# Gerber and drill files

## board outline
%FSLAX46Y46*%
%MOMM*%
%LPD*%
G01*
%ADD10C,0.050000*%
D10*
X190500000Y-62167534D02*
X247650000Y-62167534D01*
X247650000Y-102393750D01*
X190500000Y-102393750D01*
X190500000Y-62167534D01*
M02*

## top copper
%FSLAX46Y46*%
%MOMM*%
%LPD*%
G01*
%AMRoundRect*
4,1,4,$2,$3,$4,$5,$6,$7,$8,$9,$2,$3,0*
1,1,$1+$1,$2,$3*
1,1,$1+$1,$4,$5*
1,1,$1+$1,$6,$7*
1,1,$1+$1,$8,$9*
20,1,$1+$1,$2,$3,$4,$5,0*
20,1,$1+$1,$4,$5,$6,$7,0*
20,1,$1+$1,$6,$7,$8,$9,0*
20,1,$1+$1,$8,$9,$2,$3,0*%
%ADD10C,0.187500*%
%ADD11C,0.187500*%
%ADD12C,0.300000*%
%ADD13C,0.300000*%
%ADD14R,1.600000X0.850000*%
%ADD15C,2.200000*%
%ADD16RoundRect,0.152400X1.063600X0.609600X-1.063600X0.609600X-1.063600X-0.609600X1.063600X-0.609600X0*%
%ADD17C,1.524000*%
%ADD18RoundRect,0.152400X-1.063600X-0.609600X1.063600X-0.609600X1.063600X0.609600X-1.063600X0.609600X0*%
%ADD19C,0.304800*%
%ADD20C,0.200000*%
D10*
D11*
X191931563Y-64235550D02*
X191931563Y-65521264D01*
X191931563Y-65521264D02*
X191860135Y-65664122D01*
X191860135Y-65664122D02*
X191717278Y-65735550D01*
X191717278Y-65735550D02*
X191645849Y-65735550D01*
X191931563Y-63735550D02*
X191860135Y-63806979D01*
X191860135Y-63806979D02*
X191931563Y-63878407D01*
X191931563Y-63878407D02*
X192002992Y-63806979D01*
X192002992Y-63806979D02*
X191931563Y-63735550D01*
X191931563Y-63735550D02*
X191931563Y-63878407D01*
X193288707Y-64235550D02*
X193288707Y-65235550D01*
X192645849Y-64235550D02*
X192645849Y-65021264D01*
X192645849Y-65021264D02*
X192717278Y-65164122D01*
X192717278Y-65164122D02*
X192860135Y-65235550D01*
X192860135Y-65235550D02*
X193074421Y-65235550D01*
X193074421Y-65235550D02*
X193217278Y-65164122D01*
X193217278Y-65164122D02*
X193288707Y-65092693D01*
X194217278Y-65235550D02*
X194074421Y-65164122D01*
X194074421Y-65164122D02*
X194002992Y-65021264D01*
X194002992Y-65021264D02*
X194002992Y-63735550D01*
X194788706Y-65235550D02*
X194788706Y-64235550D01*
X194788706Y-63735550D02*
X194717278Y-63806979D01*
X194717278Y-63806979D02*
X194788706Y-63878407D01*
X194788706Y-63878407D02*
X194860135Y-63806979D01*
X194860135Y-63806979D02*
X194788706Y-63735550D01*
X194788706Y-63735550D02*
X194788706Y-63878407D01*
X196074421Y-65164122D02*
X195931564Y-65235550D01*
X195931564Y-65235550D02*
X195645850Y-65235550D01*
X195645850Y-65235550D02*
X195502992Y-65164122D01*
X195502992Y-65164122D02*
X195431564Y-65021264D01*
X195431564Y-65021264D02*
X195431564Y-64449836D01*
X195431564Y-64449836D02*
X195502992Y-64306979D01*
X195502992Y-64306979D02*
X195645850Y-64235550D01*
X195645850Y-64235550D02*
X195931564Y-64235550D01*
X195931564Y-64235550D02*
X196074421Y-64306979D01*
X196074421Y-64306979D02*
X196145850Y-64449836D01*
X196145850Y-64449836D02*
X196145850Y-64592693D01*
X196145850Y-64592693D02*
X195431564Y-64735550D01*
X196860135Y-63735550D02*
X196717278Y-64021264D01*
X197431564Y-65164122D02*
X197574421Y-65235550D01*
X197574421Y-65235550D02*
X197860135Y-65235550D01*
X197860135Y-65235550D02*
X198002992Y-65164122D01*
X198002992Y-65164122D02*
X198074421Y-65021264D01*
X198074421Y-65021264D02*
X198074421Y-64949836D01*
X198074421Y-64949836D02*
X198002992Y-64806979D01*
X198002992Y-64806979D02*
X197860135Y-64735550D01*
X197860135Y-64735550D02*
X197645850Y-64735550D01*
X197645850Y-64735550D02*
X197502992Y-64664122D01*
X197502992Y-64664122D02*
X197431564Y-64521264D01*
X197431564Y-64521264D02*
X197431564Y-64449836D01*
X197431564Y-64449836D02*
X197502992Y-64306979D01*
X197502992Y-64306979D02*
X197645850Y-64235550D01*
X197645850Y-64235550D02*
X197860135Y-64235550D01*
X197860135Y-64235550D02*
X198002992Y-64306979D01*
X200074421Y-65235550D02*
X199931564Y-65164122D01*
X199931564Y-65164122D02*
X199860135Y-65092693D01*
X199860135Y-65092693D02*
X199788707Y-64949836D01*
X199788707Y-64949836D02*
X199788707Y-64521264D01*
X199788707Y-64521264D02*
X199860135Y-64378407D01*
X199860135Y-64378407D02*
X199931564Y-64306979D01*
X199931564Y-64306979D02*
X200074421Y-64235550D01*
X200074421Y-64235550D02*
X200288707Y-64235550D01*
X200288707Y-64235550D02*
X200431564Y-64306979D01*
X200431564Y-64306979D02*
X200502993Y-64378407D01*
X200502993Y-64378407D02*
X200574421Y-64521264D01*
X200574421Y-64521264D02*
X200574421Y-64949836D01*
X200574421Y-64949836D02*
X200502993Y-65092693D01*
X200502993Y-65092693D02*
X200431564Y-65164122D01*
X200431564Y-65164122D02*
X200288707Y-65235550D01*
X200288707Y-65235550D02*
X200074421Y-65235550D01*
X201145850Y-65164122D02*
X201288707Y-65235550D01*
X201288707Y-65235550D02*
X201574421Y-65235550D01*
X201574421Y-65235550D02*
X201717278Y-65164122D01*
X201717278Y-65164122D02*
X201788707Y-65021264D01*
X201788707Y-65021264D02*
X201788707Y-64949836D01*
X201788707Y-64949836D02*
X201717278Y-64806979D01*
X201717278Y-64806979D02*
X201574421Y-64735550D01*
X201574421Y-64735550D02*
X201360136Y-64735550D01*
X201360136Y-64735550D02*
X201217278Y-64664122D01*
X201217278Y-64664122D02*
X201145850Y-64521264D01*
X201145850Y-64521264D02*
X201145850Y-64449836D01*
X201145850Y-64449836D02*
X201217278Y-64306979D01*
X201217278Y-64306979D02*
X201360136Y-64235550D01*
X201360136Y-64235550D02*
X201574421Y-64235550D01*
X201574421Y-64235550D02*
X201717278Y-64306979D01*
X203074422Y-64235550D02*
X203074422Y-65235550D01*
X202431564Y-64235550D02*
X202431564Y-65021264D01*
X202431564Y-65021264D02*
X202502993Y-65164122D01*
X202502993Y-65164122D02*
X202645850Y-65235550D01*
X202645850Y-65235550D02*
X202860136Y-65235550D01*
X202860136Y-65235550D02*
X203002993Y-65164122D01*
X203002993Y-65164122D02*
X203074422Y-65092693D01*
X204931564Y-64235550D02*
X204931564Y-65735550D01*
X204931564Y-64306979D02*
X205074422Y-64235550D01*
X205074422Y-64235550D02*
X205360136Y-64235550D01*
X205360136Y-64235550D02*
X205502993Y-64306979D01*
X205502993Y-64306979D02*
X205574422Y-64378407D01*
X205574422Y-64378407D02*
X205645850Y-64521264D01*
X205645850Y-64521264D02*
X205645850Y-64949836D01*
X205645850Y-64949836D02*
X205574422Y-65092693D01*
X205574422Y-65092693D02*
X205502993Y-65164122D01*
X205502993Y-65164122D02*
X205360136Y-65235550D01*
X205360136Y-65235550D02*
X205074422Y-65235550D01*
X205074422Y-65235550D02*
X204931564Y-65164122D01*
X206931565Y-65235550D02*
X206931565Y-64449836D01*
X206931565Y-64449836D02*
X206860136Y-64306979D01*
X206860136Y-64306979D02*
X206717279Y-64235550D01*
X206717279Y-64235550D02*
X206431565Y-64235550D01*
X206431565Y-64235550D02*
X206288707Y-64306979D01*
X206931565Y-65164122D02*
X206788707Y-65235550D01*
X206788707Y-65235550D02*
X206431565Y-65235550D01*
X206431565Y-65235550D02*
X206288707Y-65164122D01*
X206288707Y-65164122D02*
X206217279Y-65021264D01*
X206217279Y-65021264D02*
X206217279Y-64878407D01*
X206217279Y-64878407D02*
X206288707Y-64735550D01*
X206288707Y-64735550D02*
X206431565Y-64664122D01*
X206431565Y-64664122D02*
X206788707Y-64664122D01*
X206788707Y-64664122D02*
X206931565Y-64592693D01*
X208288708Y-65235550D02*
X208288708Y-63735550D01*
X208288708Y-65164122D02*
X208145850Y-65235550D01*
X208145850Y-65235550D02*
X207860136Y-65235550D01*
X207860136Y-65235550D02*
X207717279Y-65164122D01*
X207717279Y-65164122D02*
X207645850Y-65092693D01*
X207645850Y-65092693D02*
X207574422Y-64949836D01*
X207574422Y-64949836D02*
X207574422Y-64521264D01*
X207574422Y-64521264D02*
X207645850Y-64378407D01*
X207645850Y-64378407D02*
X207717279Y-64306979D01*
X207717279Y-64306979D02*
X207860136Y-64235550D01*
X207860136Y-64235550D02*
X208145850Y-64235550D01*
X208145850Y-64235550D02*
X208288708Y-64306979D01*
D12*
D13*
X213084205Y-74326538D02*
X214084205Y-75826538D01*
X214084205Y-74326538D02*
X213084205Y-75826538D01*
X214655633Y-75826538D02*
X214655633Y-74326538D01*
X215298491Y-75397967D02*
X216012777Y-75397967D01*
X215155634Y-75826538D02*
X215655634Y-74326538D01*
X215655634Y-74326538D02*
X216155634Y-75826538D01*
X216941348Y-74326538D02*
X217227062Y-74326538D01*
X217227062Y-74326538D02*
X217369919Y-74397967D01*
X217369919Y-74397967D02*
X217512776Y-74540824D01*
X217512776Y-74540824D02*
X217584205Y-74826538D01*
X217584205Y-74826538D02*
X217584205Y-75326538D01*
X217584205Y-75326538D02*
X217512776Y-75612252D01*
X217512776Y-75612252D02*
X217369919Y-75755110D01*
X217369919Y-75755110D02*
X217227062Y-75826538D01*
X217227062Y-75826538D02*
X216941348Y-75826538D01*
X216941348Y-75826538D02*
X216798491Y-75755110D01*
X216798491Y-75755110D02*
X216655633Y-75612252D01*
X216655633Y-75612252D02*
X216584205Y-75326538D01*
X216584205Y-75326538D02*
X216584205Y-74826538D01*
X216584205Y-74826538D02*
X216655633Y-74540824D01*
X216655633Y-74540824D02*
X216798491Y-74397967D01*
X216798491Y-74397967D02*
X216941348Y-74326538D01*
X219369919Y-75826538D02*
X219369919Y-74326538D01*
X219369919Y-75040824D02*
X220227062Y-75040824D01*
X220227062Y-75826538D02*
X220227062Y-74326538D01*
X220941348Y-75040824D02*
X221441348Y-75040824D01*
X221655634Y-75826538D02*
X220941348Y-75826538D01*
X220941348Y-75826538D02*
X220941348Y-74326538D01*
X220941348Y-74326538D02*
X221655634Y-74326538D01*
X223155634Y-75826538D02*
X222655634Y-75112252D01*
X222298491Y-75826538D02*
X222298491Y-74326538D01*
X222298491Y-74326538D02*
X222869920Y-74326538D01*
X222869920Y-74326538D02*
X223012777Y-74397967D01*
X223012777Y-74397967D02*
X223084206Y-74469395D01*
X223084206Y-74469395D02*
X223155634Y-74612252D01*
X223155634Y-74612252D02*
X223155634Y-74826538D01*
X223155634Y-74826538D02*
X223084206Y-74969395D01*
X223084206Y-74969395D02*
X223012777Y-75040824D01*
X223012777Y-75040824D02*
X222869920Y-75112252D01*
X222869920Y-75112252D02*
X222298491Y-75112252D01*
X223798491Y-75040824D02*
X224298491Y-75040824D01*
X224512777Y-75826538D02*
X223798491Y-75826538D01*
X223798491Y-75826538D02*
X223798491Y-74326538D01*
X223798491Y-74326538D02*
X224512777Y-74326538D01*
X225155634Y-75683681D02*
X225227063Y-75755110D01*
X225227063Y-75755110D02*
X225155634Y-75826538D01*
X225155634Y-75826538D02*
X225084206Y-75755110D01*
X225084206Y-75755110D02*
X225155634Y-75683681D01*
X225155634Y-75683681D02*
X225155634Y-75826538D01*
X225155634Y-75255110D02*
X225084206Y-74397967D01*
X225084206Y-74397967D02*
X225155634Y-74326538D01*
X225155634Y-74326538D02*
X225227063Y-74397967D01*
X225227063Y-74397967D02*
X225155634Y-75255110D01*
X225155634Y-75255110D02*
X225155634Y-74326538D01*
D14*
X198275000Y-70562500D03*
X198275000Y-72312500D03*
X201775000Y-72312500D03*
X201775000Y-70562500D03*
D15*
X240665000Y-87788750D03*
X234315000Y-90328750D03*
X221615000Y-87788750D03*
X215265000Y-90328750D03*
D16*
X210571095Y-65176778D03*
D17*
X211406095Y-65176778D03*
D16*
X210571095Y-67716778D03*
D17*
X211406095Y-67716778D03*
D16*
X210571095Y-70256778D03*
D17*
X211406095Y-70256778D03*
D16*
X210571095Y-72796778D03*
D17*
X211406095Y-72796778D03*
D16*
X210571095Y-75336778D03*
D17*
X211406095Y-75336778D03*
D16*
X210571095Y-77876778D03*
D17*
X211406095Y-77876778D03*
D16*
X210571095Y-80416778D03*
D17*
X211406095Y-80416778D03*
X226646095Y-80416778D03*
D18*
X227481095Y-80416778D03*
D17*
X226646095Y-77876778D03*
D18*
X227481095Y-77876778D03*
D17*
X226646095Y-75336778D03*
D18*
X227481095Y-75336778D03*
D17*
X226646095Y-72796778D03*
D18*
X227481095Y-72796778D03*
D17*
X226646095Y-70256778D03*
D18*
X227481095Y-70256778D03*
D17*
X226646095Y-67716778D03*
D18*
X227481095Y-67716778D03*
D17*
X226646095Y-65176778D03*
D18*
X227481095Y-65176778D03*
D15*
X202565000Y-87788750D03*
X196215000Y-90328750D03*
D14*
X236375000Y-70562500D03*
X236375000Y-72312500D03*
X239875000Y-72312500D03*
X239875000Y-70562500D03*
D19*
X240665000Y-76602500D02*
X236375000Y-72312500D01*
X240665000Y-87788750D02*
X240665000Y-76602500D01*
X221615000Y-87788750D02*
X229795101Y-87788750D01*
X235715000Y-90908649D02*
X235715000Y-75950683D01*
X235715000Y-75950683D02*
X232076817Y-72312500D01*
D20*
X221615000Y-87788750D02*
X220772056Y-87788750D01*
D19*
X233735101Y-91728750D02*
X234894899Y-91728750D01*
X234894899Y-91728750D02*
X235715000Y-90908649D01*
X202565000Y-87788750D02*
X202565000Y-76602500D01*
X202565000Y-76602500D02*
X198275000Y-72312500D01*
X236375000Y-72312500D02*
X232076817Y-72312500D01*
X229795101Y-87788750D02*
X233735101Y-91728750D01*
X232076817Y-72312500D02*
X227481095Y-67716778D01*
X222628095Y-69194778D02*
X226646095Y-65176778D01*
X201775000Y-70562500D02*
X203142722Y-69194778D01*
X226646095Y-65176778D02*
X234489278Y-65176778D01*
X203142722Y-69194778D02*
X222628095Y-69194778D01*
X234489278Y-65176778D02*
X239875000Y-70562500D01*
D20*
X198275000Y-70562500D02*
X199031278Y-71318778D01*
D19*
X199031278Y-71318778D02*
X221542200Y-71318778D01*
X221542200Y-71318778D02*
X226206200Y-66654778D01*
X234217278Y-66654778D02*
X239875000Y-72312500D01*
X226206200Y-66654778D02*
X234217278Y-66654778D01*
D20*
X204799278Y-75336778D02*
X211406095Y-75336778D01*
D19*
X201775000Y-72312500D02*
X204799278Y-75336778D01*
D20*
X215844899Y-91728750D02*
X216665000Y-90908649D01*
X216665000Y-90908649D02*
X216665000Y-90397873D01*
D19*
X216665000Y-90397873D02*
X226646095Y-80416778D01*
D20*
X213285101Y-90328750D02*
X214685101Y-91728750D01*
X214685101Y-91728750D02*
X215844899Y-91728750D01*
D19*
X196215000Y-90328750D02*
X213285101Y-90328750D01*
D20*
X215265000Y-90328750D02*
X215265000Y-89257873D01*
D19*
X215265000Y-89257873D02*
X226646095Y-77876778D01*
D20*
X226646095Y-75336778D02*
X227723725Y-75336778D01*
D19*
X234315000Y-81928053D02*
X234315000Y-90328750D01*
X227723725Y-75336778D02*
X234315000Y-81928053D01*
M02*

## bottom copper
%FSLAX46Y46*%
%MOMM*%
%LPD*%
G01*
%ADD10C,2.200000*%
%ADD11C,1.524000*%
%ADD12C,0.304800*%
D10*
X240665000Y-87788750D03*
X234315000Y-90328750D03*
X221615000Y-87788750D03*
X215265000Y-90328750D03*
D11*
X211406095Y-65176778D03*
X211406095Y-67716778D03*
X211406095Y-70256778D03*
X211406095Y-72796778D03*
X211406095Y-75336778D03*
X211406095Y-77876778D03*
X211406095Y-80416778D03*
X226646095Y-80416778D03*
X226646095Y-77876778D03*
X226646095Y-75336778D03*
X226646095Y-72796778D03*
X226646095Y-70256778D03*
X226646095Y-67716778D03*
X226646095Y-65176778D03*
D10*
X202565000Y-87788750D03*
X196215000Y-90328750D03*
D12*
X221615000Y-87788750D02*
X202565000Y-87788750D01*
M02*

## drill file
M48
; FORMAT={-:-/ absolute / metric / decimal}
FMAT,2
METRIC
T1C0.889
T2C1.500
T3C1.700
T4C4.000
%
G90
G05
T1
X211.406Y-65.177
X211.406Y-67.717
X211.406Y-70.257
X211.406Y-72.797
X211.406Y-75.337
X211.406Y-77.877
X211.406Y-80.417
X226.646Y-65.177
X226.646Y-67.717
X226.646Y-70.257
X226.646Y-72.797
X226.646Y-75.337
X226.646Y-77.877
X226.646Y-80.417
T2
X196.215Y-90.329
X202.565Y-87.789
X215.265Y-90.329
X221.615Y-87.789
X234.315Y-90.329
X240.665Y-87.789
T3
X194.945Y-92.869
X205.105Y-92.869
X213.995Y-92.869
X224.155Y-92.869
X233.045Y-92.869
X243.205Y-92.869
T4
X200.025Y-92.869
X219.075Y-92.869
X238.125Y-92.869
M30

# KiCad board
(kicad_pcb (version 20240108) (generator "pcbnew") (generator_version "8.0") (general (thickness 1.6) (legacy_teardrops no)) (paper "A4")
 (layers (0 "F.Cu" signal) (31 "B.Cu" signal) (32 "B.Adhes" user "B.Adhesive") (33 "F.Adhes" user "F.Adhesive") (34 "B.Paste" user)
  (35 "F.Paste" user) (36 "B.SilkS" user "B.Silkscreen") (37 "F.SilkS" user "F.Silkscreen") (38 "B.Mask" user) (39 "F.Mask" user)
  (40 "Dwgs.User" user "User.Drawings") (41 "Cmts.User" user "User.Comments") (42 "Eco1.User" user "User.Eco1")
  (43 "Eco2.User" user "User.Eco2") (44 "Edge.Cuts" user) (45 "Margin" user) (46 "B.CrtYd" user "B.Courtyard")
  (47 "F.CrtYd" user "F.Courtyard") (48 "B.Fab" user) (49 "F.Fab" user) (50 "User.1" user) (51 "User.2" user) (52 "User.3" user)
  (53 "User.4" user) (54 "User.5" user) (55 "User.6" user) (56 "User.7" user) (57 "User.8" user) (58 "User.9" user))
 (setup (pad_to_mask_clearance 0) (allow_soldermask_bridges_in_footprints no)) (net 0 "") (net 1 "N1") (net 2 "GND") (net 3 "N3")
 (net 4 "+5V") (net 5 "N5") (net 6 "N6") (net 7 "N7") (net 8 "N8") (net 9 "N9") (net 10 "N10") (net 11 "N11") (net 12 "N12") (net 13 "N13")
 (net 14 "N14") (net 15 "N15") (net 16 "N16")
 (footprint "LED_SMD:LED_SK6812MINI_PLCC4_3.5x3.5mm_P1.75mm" (layer "F.Cu") (at 200.025 71.4375)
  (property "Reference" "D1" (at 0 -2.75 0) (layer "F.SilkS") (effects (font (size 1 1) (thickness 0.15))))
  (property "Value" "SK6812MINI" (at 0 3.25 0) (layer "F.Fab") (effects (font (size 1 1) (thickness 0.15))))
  (pad "1" smd rect (at -1.75 -0.875) (size 1.6 0.85) (layers "F.Cu" "F.Paste" "F.Mask") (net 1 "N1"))
  (pad "2" smd rect (at -1.75 0.875) (size 1.6 0.85) (layers "F.Cu" "F.Paste" "F.Mask") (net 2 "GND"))
  (pad "3" smd rect (at 1.75 0.875) (size 1.6 0.85) (layers "F.Cu" "F.Paste" "F.Mask") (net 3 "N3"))
  (pad "4" smd rect (at 1.75 -0.875) (size 1.6 0.85) (layers "F.Cu" "F.Paste" "F.Mask") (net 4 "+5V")))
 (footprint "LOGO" (layer "F.Cu") (at 219.075 76.2)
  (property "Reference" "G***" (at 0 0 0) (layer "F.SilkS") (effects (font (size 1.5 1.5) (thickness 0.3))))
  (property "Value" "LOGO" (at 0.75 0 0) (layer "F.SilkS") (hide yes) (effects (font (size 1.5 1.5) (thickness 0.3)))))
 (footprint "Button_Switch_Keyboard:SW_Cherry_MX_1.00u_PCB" (layer "F.Cu") (at 240.665 87.78875)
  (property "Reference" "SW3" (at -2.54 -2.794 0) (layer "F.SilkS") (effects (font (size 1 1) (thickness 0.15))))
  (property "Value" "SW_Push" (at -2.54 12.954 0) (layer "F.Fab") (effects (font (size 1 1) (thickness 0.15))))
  (pad "" np_thru_hole circle (at -7.62 5.08) (size 1.7 1.7) (drill 1.7) (layers "*.Cu" "*.Mask"))
  (pad "" np_thru_hole circle (at -2.54 5.08) (size 4 4) (drill 4) (layers "*.Cu" "*.Mask"))
  (pad "" np_thru_hole circle (at 2.54 5.08) (size 1.7 1.7) (drill 1.7) (layers "*.Cu" "*.Mask"))
  (pad "1" thru_hole circle (at 0 0) (size 2.2 2.2) (drill 1.5) (layers "*.Cu" "*.Mask") (remove_unused_layers no) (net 2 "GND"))
  (pad "2" thru_hole circle (at -6.35 2.54) (size 2.2 2.2) (drill 1.5) (layers "*.Cu" "*.Mask") (remove_unused_layers no) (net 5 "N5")))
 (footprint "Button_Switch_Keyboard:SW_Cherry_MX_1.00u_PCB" (layer "F.Cu") (at 221.615 87.78875)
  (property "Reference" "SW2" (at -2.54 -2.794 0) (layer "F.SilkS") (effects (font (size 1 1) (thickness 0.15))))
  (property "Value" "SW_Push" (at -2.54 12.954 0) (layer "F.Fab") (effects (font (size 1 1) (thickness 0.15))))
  (pad "" np_thru_hole circle (at -7.62 5.08) (size 1.7 1.7) (drill 1.7) (layers "*.Cu" "*.Mask"))
  (pad "" np_thru_hole circle (at -2.54 5.08) (size 4 4) (drill 4) (layers "*.Cu" "*.Mask"))
  (pad "" np_thru_hole circle (at 2.54 5.08) (size 1.7 1.7) (drill 1.7) (layers "*.Cu" "*.Mask"))
  (pad "1" thru_hole circle (at 0 0) (size 2.2 2.2) (drill 1.5) (layers "*.Cu" "*.Mask") (remove_unused_layers no) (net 2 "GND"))
  (pad "2" thru_hole circle (at -6.35 2.54) (size 2.2 2.2) (drill 1.5) (layers "*.Cu" "*.Mask") (remove_unused_layers no) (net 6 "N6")))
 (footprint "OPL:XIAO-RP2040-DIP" (layer "F.Cu") (at 219.026095 72.796778)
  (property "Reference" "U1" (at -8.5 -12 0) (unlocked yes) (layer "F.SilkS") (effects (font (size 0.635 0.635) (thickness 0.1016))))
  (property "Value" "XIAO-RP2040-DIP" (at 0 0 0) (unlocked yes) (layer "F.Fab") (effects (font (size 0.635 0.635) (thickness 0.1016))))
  (pad "1" smd roundrect (at -8.455 -7.62 180) (size 2.432 1.524) (layers "F.Cu" "F.Mask") (roundrect_rratio 0.1) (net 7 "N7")
   (thermal_bridge_angle 45))
  (pad "1" thru_hole circle (at -7.62 -7.62 180) (size 1.524 1.524) (drill 0.889) (layers "*.Cu" "*.Mask") (remove_unused_layers no)
   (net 7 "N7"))
  (pad "2" smd roundrect (at -8.455 -5.08 180) (size 2.432 1.524) (layers "F.Cu" "F.Mask") (roundrect_rratio 0.1) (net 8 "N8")
   (thermal_bridge_angle 45))
  (pad "2" thru_hole circle (at -7.62 -5.08 180) (size 1.524 1.524) (drill 0.889) (layers "*.Cu" "*.Mask") (remove_unused_layers no)
   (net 8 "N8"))
  (pad "3" smd roundrect (at -8.455 -2.54 180) (size 2.432 1.524) (layers "F.Cu" "F.Mask") (roundrect_rratio 0.1) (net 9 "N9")
   (thermal_bridge_angle 45))
  (pad "3" thru_hole circle (at -7.62 -2.54 180) (size 1.524 1.524) (drill 0.889) (layers "*.Cu" "*.Mask") (remove_unused_layers no)
   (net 9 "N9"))
  (pad "4" smd roundrect (at -8.455 0 180) (size 2.432 1.524) (layers "F.Cu" "F.Mask") (roundrect_rratio 0.1) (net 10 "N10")
   (thermal_bridge_angle 45))
  (pad "4" thru_hole circle (at -7.62 0 180) (size 1.524 1.524) (drill 0.889) (layers "*.Cu" "*.Mask") (remove_unused_layers no)
   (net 10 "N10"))
  (pad "5" smd roundrect (at -8.455 2.54 180) (size 2.432 1.524) (layers "F.Cu" "F.Mask") (roundrect_rratio 0.1) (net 3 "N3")
   (thermal_bridge_angle 45))
  (pad "5" thru_hole circle (at -7.62 2.54 180) (size 1.524 1.524) (drill 0.889) (layers "*.Cu" "*.Mask") (remove_unused_layers no)
   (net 3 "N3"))
  (pad "6" smd roundrect (at -8.455 5.08 180) (size 2.432 1.524) (layers "F.Cu" "F.Mask") (roundrect_rratio 0.1) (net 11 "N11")
   (thermal_bridge_angle 45))
  (pad "6" thru_hole circle (at -7.62 5.08 180) (size 1.524 1.524) (drill 0.889) (layers "*.Cu" "*.Mask") (remove_unused_layers no)
   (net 11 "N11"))
  (pad "7" smd roundrect (at -8.455 7.62 180) (size 2.432 1.524) (layers "F.Cu" "F.Mask") (roundrect_rratio 0.1) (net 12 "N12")
   (thermal_bridge_angle 45))
  (pad "7" thru_hole circle (at -7.62 7.62 180) (size 1.524 1.524) (drill 0.889) (layers "*.Cu" "*.Mask") (remove_unused_layers no)
   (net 12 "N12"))
  (pad "8" thru_hole circle (at 7.62 7.62) (size 1.524 1.524) (drill 0.889) (layers "*.Cu" "*.Mask") (remove_unused_layers no)
   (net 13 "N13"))
  (pad "8" smd roundrect (at 8.455 7.62) (size 2.432 1.524) (layers "F.Cu" "F.Mask") (roundrect_rratio 0.1) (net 13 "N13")
   (thermal_bridge_angle 45))
  (pad "9" thru_hole circle (at 7.62 5.08) (size 1.524 1.524) (drill 0.889) (layers "*.Cu" "*.Mask") (remove_unused_layers no) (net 6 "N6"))
  (pad "9" smd roundrect (at 8.455 5.08) (size 2.432 1.524) (layers "F.Cu" "F.Mask") (roundrect_rratio 0.1) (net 6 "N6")
   (thermal_bridge_angle 45))
  (pad "10" thru_hole circle (at 7.62 2.54) (size 1.524 1.524) (drill 0.889) (layers "*.Cu" "*.Mask") (remove_unused_layers no) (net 5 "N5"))
  (pad "10" smd roundrect (at 8.455 2.54) (size 2.432 1.524) (layers "F.Cu" "F.Mask") (roundrect_rratio 0.1) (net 5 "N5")
   (thermal_bridge_angle 45))
  (pad "11" thru_hole circle (at 7.62 0) (size 1.524 1.524) (drill 0.889) (layers "*.Cu" "*.Mask") (remove_unused_layers no) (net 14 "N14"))
  (pad "11" smd roundrect (at 8.455 0) (size 2.432 1.524) (layers "F.Cu" "F.Mask") (roundrect_rratio 0.1) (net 14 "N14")
   (thermal_bridge_angle 45))
  (pad "12" thru_hole circle (at 7.62 -2.54) (size 1.524 1.524) (drill 0.889) (layers "*.Cu" "*.Mask") (remove_unused_layers no)
   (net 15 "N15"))
  (pad "12" smd roundrect (at 8.455 -2.54) (size 2.432 1.524) (layers "F.Cu" "F.Mask") (roundrect_rratio 0.1) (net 15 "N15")
   (thermal_bridge_angle 45))
  (pad "13" thru_hole circle (at 7.62 -5.08) (size 1.524 1.524) (drill 0.889) (layers "*.Cu" "*.Mask") (remove_unused_layers no)
   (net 2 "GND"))
  (pad "13" smd roundrect (at 8.455 -5.08) (size 2.432 1.524) (layers "F.Cu" "F.Mask") (roundrect_rratio 0.1) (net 2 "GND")
   (thermal_bridge_angle 45))
  (pad "14" thru_hole circle (at 7.62 -7.62) (size 1.524 1.524) (drill 0.889) (layers "*.Cu" "*.Mask") (remove_unused_layers no)
   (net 4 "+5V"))
  (pad "14" smd roundrect (at 8.455 -7.62) (size 2.432 1.524) (layers "F.Cu" "F.Mask") (roundrect_rratio 0.1) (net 4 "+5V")
   (thermal_bridge_angle 45)))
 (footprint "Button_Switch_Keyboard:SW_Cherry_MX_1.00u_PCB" (layer "F.Cu") (at 202.565 87.78875)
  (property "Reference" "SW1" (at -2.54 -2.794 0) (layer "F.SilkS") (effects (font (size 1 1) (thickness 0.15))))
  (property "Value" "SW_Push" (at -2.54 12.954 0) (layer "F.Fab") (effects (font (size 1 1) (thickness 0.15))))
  (pad "" np_thru_hole circle (at -7.62 5.08) (size 1.7 1.7) (drill 1.7) (layers "*.Cu" "*.Mask"))
  (pad "" np_thru_hole circle (at -2.54 5.08) (size 4 4) (drill 4) (layers "*.Cu" "*.Mask"))
  (pad "" np_thru_hole circle (at 2.54 5.08) (size 1.7 1.7) (drill 1.7) (layers "*.Cu" "*.Mask"))
  (pad "1" thru_hole circle (at 0 0) (size 2.2 2.2) (drill 1.5) (layers "*.Cu" "*.Mask") (remove_unused_layers no) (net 2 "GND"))
  (pad "2" thru_hole circle (at -6.35 2.54) (size 2.2 2.2) (drill 1.5) (layers "*.Cu" "*.Mask") (remove_unused_layers no) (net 13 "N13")))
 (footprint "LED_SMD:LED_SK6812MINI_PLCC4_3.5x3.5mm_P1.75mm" (layer "F.Cu") (at 238.125 71.4375)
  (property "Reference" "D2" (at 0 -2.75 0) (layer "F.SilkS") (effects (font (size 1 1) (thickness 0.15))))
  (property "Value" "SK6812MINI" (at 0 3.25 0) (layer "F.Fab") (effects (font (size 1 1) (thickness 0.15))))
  (pad "1" smd rect (at -1.75 -0.875) (size 1.6 0.85) (layers "F.Cu" "F.Paste" "F.Mask") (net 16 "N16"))
  (pad "2" smd rect (at -1.75 0.875) (size 1.6 0.85) (layers "F.Cu" "F.Paste" "F.Mask") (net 2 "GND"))
  (pad "3" smd rect (at 1.75 0.875) (size 1.6 0.85) (layers "F.Cu" "F.Paste" "F.Mask") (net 1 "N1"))
  (pad "4" smd rect (at 1.75 -0.875) (size 1.6 0.85) (layers "F.Cu" "F.Paste" "F.Mask") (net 4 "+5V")))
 (gr_rect (start 190.5 62.167534) (end 247.65 102.39375) (stroke (width 0.05) (type default)) (fill none) (layer "Edge.Cuts"))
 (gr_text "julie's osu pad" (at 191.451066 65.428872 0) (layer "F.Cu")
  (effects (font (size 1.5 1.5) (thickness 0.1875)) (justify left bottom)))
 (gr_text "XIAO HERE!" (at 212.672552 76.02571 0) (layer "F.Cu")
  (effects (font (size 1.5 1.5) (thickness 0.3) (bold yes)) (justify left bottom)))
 (segment (start 240.665 76.6025) (end 236.375 72.3125) (width 0.3048) (layer "F.Cu") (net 2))
 (segment (start 240.665 87.78875) (end 240.665 76.6025) (width 0.3048) (layer "F.Cu") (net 2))
 (segment (start 221.615 87.78875) (end 229.795101 87.78875) (width 0.3048) (layer "F.Cu") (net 2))
 (segment (start 235.715 90.908649) (end 235.715 75.950683) (width 0.3048) (layer "F.Cu") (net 2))
 (segment (start 235.715 75.950683) (end 232.076817 72.3125) (width 0.3048) (layer "F.Cu") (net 2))
 (segment (start 221.615 87.78875) (end 220.772056 87.78875) (width 0.2) (layer "F.Cu") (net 2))
 (segment (start 233.735101 91.72875) (end 234.894899 91.72875) (width 0.3048) (layer "F.Cu") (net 2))
 (segment (start 234.894899 91.72875) (end 235.715 90.908649) (width 0.3048) (layer "F.Cu") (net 2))
 (segment (start 202.565 87.78875) (end 202.565 76.6025) (width 0.3048) (layer "F.Cu") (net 2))
 (segment (start 202.565 76.6025) (end 198.275 72.3125) (width 0.3048) (layer "F.Cu") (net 2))
 (segment (start 236.375 72.3125) (end 232.076817 72.3125) (width 0.3048) (layer "F.Cu") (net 2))
 (segment (start 229.795101 87.78875) (end 233.735101 91.72875) (width 0.3048) (layer "F.Cu") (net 2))
 (segment (start 232.076817 72.3125) (end 227.481095 67.716778) (width 0.3048) (layer "F.Cu") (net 2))
 (segment (start 221.615 87.78875) (end 202.565 87.78875) (width 0.3048) (layer "B.Cu") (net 2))
 (segment (start 222.628095 69.194778) (end 226.646095 65.176778) (width 0.3048) (layer "F.Cu") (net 4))
 (segment (start 201.775 70.5625) (end 203.142722 69.194778) (width 0.3048) (layer "F.Cu") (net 4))
 (segment (start 226.646095 65.176778) (end 234.489278 65.176778) (width 0.3048) (layer "F.Cu") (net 4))
 (segment (start 203.142722 69.194778) (end 222.628095 69.194778) (width 0.3048) (layer "F.Cu") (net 4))
 (segment (start 234.489278 65.176778) (end 239.875 70.5625) (width 0.3048) (layer "F.Cu") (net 4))
 (segment (start 198.275 70.5625) (end 199.031278 71.318778) (width 0.2) (layer "F.Cu") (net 1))
 (segment (start 199.031278 71.318778) (end 221.5422 71.318778) (width 0.3048) (layer "F.Cu") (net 1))
 (segment (start 221.5422 71.318778) (end 226.2062 66.654778) (width 0.3048) (layer "F.Cu") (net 1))
 (segment (start 234.217278 66.654778) (end 239.875 72.3125) (width 0.3048) (layer "F.Cu") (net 1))
 (segment (start 226.2062 66.654778) (end 234.217278 66.654778) (width 0.3048) (layer "F.Cu") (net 1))
 (segment (start 204.799278 75.336778) (end 211.406095 75.336778) (width 0.2) (layer "F.Cu") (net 3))
 (segment (start 201.775 72.3125) (end 204.799278 75.336778) (width 0.3048) (layer "F.Cu") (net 3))
 (segment (start 215.844899 91.72875) (end 216.665 90.908649) (width 0.2) (layer "F.Cu") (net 13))
 (segment (start 216.665 90.908649) (end 216.665 90.397873) (width 0.2) (layer "F.Cu") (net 13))
 (segment (start 216.665 90.397873) (end 226.646095 80.416778) (width 0.3048) (layer "F.Cu") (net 13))
 (segment (start 213.285101 90.32875) (end 214.685101 91.72875) (width 0.2) (layer "F.Cu") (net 13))
 (segment (start 214.685101 91.72875) (end 215.844899 91.72875) (width 0.2) (layer "F.Cu") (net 13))
 (segment (start 196.215 90.32875) (end 213.285101 90.32875) (width 0.3048) (layer "F.Cu") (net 13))
 (segment (start 215.265 90.32875) (end 215.265 89.257873) (width 0.2) (layer "F.Cu") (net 6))
 (segment (start 215.265 89.257873) (end 226.646095 77.876778) (width 0.3048) (layer "F.Cu") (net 6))
 (segment (start 226.646095 75.336778) (end 227.723725 75.336778) (width 0.2) (layer "F.Cu") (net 5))
 (segment (start 234.315 81.928053) (end 234.315 90.32875) (width 0.3048) (layer "F.Cu") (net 5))
 (segment (start 227.723725 75.336778) (end 234.315 81.928053) (width 0.3048) (layer "F.Cu") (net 5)))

